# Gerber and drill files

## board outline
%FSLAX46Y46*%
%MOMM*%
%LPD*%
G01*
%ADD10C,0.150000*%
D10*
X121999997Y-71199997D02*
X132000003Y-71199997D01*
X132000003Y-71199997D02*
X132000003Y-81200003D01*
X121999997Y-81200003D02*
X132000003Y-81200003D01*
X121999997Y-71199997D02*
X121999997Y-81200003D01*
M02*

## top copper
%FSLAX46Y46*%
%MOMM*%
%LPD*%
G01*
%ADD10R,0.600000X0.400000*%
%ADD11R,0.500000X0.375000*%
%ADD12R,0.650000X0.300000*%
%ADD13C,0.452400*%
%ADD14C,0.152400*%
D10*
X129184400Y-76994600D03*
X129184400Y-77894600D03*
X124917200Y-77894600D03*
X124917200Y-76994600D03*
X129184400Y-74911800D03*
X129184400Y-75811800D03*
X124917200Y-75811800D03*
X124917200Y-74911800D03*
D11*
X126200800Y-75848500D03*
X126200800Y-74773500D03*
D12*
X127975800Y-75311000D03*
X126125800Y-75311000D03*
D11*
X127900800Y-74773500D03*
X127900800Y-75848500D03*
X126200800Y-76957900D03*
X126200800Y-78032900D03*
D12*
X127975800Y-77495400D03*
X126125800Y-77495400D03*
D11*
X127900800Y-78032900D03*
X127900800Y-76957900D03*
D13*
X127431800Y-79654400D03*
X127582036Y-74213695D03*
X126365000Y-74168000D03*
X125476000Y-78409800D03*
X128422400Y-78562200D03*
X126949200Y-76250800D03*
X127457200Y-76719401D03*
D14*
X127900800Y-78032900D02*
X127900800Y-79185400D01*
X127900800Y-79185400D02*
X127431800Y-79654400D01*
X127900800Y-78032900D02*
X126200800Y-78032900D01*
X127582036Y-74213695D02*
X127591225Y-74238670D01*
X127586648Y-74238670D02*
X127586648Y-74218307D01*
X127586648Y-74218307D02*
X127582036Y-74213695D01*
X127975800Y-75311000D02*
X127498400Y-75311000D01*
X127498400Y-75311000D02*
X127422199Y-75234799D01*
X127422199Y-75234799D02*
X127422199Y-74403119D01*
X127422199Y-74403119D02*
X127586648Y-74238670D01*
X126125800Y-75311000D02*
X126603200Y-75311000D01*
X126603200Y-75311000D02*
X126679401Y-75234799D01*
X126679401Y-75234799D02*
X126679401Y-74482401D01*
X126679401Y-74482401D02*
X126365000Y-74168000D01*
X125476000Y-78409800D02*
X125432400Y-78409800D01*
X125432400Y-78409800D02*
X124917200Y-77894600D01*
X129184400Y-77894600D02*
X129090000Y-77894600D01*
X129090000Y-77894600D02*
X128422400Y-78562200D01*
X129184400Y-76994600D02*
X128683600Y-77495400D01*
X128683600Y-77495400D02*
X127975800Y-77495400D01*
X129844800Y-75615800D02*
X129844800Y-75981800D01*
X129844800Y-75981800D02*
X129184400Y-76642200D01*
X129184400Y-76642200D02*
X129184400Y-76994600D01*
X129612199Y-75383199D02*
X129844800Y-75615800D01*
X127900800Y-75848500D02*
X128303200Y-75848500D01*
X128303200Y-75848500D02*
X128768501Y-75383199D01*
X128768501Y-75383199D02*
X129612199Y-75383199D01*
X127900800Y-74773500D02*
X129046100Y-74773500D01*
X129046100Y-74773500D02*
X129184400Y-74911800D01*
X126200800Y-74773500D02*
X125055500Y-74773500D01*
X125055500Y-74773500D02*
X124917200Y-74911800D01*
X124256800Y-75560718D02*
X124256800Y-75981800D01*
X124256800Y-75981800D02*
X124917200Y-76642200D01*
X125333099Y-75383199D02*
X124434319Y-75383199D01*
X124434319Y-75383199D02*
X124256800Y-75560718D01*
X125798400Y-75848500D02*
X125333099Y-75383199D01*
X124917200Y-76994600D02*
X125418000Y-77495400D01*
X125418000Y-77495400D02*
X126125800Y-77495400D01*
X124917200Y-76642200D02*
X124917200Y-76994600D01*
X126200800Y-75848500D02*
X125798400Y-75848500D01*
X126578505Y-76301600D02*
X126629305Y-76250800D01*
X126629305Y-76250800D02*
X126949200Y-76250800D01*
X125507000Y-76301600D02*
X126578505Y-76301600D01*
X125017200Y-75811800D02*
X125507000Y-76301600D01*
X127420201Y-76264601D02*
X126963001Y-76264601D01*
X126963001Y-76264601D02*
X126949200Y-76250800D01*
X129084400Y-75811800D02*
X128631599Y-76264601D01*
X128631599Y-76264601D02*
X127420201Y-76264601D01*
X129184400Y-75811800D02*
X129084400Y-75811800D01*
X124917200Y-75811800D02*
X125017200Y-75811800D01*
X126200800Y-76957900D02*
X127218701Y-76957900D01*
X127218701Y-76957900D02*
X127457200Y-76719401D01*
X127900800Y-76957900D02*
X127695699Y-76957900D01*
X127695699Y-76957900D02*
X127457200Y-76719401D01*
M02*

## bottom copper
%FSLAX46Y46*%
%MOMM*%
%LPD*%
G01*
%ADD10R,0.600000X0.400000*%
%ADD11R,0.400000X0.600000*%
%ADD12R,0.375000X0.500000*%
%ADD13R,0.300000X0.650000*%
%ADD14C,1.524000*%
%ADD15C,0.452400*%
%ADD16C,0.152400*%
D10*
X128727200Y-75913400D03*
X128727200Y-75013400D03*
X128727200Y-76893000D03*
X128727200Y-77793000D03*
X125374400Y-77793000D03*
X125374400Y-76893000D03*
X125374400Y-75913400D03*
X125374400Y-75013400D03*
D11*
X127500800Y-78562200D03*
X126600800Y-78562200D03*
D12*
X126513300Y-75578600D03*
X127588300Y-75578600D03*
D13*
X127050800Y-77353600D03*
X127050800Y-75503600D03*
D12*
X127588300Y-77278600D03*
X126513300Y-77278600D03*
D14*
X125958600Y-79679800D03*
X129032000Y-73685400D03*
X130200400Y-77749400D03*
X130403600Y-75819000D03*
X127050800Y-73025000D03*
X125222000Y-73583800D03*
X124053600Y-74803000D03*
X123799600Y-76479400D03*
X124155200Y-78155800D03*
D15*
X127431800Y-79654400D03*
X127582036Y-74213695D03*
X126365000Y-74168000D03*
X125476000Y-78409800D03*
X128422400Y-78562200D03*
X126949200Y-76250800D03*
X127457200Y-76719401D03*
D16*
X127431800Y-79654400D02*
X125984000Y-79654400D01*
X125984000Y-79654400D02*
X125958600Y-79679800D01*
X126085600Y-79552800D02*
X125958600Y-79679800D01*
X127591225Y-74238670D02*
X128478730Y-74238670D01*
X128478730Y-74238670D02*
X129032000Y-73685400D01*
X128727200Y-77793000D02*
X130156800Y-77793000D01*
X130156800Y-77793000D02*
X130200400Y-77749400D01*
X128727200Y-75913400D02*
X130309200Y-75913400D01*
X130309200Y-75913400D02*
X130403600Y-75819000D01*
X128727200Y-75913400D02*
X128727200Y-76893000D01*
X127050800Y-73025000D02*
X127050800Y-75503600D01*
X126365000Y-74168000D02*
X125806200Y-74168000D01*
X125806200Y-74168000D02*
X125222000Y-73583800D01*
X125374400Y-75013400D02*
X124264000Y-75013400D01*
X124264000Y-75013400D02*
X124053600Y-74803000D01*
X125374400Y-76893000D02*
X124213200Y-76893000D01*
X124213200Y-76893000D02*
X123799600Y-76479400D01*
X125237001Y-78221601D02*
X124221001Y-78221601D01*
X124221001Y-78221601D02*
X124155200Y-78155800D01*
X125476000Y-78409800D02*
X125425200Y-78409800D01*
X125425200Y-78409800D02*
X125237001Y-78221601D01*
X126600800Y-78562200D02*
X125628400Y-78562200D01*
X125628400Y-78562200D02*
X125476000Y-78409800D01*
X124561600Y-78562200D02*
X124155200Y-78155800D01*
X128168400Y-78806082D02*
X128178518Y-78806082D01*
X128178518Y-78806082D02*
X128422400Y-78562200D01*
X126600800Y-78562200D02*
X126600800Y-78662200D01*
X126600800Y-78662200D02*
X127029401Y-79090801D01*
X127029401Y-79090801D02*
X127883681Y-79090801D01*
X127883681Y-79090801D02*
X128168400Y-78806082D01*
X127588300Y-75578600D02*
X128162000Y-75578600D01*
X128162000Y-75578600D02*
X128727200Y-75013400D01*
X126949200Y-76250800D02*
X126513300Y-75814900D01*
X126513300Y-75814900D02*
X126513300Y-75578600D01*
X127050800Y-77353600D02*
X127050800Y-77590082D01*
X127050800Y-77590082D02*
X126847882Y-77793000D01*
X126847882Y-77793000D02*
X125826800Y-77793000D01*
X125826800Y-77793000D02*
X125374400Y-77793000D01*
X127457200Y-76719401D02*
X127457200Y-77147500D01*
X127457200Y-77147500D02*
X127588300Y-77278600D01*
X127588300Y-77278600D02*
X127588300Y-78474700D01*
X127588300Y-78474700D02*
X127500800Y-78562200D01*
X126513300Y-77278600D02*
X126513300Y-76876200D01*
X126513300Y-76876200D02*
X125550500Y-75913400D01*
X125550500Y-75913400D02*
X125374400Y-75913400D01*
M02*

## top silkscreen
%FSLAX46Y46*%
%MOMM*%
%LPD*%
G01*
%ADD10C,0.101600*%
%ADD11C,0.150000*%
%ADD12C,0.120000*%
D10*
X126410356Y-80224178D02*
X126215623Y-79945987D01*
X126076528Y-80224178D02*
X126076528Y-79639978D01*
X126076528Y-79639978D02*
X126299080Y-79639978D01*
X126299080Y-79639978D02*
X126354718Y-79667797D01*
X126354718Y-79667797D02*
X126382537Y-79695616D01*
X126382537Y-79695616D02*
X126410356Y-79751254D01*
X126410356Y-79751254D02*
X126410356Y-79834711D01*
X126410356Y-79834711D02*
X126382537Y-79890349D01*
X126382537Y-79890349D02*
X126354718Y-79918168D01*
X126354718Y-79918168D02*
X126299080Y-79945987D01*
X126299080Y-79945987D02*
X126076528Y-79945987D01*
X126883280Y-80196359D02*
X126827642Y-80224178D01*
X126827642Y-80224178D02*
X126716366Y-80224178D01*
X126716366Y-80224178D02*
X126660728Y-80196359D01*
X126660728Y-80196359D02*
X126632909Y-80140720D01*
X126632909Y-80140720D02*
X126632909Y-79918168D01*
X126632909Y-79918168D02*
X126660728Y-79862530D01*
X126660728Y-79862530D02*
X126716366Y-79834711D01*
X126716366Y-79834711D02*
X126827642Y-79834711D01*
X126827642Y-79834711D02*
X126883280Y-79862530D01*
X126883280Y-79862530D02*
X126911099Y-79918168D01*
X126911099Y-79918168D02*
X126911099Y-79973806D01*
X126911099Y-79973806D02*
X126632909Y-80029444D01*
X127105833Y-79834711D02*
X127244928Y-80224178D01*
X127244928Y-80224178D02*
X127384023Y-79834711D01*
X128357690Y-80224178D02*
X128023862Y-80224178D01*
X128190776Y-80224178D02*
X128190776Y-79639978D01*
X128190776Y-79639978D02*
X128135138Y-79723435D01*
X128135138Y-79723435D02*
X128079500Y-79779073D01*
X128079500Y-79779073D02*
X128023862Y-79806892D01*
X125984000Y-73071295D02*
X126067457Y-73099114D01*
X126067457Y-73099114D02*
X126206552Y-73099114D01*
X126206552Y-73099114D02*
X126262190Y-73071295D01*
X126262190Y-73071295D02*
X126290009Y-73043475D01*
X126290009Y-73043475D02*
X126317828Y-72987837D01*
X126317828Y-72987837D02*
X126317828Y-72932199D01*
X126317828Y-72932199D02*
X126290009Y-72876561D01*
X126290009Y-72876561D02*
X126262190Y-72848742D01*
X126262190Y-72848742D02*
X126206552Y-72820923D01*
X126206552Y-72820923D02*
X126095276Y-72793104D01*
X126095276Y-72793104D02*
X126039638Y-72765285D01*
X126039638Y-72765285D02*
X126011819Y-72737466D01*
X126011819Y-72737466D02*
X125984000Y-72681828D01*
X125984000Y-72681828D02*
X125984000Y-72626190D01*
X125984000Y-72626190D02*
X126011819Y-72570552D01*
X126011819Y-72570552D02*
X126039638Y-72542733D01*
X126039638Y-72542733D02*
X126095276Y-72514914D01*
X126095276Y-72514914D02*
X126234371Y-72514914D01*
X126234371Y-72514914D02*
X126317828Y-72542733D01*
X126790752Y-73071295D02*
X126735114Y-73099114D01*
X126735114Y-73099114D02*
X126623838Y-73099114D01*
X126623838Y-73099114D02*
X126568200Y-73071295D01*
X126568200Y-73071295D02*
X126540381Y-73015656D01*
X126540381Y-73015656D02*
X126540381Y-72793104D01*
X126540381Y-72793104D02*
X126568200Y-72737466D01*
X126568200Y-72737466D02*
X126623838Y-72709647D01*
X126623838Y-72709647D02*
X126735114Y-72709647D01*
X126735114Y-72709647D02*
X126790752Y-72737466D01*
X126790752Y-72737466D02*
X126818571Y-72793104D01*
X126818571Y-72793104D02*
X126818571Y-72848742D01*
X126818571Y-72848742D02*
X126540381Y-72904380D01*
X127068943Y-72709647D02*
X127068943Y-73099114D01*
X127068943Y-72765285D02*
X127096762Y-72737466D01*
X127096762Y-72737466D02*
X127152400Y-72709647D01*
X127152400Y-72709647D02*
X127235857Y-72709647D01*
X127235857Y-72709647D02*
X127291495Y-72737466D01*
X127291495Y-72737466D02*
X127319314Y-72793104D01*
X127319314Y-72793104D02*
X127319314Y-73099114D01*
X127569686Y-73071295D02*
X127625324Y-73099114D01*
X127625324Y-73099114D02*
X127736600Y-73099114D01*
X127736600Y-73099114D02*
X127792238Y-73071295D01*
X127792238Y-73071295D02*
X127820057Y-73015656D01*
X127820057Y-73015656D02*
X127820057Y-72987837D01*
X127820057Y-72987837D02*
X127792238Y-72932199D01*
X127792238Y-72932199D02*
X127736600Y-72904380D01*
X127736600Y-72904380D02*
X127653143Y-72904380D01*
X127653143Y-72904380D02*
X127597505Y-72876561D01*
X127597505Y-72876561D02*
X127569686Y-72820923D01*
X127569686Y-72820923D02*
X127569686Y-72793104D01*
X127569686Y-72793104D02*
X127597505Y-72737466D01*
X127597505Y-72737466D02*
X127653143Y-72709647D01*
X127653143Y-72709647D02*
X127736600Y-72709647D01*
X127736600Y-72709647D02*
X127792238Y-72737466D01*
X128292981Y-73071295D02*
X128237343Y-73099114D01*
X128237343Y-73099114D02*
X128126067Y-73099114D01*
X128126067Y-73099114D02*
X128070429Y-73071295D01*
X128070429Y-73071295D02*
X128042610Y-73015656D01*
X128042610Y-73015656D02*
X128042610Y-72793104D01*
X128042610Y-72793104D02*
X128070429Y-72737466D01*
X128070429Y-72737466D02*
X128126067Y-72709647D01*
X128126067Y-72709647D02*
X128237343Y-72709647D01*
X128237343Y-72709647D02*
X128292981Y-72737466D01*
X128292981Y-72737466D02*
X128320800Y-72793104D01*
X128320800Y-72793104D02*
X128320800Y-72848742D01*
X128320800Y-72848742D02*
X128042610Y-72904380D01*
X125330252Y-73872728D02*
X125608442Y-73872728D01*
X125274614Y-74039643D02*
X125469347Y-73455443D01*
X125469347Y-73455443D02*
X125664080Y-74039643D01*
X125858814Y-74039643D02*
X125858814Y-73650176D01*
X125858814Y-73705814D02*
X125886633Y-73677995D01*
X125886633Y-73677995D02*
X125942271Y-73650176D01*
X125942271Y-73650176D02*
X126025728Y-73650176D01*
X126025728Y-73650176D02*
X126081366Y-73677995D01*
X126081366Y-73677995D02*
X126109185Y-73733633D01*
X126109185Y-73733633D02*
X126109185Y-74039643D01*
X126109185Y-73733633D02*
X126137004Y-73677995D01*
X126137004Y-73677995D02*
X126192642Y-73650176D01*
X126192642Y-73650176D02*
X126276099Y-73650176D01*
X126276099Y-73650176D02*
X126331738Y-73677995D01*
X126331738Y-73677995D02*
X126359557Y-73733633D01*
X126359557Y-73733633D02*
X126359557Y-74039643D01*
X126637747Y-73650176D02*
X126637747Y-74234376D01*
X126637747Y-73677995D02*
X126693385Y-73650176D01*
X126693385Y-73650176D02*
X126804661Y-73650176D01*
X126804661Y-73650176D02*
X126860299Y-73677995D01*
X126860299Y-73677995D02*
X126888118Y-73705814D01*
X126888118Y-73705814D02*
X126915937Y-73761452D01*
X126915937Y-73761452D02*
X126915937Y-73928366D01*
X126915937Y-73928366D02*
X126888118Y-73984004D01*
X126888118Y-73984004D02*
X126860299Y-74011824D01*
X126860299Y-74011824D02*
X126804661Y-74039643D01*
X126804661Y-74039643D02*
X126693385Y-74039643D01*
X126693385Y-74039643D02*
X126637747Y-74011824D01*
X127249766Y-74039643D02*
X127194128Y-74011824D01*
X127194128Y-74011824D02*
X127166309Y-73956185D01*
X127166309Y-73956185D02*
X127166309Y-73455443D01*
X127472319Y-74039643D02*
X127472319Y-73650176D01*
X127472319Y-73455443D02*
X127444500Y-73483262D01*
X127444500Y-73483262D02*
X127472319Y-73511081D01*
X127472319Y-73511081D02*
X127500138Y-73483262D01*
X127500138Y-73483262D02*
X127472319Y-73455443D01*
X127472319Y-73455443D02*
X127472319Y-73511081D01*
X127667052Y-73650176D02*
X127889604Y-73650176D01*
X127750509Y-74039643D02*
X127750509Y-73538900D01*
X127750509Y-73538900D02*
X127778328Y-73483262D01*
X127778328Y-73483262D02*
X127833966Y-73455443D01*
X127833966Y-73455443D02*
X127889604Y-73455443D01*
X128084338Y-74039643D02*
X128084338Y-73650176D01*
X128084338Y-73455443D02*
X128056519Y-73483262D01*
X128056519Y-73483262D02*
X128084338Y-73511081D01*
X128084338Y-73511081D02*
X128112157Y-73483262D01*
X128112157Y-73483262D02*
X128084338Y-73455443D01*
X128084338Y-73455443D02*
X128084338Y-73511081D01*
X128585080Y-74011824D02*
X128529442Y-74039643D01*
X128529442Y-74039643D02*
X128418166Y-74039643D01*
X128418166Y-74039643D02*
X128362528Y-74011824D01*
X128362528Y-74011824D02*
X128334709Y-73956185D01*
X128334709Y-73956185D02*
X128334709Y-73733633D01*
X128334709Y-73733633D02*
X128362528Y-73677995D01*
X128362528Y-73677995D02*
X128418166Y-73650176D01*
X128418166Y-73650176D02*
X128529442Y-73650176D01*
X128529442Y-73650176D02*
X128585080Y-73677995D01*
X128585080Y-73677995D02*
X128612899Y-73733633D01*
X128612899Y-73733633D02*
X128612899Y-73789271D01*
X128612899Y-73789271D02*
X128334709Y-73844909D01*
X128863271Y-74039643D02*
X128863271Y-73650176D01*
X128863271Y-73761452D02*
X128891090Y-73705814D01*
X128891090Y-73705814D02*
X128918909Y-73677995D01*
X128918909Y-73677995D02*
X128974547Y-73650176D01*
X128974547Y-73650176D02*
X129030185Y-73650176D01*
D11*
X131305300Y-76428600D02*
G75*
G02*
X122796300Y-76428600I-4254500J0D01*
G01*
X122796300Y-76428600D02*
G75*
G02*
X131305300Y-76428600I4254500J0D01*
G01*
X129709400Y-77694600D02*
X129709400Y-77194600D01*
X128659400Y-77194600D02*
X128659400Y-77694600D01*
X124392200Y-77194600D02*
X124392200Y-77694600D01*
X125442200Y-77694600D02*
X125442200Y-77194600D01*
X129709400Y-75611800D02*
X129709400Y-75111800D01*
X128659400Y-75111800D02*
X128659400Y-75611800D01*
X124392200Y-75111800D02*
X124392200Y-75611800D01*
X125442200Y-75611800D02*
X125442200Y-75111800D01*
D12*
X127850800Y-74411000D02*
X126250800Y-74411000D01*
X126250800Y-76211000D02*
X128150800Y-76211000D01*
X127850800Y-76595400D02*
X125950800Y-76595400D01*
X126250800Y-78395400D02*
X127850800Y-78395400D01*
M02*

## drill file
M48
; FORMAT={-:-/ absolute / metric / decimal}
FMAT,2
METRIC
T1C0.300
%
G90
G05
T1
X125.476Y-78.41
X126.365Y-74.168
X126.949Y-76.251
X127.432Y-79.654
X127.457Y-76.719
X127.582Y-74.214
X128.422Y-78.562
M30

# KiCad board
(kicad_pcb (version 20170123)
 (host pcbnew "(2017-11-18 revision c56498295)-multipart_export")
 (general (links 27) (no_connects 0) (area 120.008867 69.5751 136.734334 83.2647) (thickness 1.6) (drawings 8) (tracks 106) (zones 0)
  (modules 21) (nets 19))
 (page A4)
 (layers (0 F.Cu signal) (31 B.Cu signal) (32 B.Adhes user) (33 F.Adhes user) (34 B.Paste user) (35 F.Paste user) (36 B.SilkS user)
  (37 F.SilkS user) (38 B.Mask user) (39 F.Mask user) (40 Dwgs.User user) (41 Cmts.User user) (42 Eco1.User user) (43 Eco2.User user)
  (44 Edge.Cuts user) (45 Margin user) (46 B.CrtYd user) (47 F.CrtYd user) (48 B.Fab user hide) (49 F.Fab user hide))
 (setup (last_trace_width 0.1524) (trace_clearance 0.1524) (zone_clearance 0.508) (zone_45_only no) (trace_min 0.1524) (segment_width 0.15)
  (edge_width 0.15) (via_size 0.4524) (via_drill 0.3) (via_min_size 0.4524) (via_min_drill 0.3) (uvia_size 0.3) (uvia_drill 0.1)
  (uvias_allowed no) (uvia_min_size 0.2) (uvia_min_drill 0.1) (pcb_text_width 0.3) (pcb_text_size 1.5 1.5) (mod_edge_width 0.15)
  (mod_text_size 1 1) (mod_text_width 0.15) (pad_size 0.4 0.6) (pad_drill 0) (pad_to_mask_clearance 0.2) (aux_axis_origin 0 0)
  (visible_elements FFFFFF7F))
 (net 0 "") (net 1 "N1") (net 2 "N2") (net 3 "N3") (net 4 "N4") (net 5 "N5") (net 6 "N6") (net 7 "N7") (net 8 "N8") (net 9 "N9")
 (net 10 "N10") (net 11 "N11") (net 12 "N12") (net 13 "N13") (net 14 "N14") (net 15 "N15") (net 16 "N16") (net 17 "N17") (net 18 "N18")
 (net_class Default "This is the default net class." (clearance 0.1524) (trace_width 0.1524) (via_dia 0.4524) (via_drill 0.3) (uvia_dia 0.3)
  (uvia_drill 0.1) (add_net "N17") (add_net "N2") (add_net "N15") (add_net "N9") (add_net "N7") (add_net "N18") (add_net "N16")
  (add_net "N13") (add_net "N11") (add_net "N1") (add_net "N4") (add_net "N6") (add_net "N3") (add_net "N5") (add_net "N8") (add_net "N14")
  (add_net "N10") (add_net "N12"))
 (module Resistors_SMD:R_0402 (layer F.Cu) (at 129.1844 77.4446 90)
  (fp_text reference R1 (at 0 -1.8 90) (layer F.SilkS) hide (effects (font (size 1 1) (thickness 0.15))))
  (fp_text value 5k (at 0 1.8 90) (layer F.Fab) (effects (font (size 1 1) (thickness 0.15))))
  (fp_line (start -0.25 0.525) (end 0.25 0.525) (layer F.SilkS) (width 0.15))
  (fp_line (start 0.25 -0.525) (end -0.25 -0.525) (layer F.SilkS) (width 0.15))
  (pad 2 smd rect (at 0.45 0 90) (size 0.4 0.6) (layers F.Cu F.Paste F.Mask) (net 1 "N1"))
  (pad 1 smd rect (at -0.45 0 90) (size 0.4 0.6) (layers F.Cu F.Paste F.Mask) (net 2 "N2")))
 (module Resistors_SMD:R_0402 (layer F.Cu) (at 124.9172 77.4446 90)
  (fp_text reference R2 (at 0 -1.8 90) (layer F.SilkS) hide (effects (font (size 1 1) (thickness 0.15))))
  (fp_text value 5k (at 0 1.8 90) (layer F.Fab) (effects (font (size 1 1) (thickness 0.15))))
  (fp_line (start 0.25 -0.525) (end -0.25 -0.525) (layer F.SilkS) (width 0.15))
  (fp_line (start -0.25 0.525) (end 0.25 0.525) (layer F.SilkS) (width 0.15))
  (pad 1 smd rect (at -0.45 0 90) (size 0.4 0.6) (layers F.Cu F.Paste F.Mask) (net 2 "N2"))
  (pad 2 smd rect (at 0.45 0 90) (size 0.4 0.6) (layers F.Cu F.Paste F.Mask) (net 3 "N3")))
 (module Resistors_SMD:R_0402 (layer F.Cu) (at 129.1844 75.3618 270)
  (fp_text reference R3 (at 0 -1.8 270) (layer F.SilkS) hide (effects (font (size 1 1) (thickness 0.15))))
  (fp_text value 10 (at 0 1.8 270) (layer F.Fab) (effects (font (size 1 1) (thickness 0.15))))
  (fp_line (start 0.25 -0.525) (end -0.25 -0.525) (layer F.SilkS) (width 0.15))
  (fp_line (start -0.25 0.525) (end 0.25 0.525) (layer F.SilkS) (width 0.15))
  (pad 1 smd rect (at -0.45 0 270) (size 0.4 0.6) (layers F.Cu F.Paste F.Mask) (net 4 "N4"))
  (pad 2 smd rect (at 0.45 0 270) (size 0.4 0.6) (layers F.Cu F.Paste F.Mask) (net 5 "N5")))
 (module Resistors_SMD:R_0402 (layer F.Cu) (at 124.9172 75.3618 270)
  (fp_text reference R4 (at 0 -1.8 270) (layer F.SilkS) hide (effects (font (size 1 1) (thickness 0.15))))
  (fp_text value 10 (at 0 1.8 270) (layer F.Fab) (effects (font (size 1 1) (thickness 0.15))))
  (fp_line (start -0.25 0.525) (end 0.25 0.525) (layer F.SilkS) (width 0.15))
  (fp_line (start 0.25 -0.525) (end -0.25 -0.525) (layer F.SilkS) (width 0.15))
  (pad 2 smd rect (at 0.45 0 270) (size 0.4 0.6) (layers F.Cu F.Paste F.Mask) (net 5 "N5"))
  (pad 1 smd rect (at -0.45 0 270) (size 0.4 0.6) (layers F.Cu F.Paste F.Mask) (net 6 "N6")))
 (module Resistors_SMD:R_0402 (layer B.Cu) (at 128.7272 75.4634 270)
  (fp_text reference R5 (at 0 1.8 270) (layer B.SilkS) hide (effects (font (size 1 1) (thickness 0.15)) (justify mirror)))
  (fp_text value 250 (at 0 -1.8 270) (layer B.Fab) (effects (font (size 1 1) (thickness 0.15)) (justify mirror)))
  (pad 2 smd rect (at 0.45 0 270) (size 0.4 0.6) (layers B.Cu B.Paste B.Mask) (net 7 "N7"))
  (pad 1 smd rect (at -0.45 0 270) (size 0.4 0.6) (layers B.Cu B.Paste B.Mask) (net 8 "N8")))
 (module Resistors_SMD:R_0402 (layer B.Cu) (at 128.7272 77.343 270)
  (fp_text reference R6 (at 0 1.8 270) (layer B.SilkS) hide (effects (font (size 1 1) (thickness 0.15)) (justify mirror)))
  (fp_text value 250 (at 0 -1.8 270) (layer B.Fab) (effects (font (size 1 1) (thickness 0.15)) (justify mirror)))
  (pad 1 smd rect (at -0.45 0 270) (size 0.4 0.6) (layers B.Cu B.Paste B.Mask) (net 7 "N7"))
  (pad 2 smd rect (at 0.45 0 270) (size 0.4 0.6) (layers B.Cu B.Paste B.Mask) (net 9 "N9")))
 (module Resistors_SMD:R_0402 (layer B.Cu) (at 125.3744 77.343 90)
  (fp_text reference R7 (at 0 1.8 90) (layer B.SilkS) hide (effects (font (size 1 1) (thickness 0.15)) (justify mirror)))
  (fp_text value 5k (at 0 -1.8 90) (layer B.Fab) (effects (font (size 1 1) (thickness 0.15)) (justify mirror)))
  (pad 1 smd rect (at -0.45 0 90) (size 0.4 0.6) (layers B.Cu B.Paste B.Mask) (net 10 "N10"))
  (pad 2 smd rect (at 0.45 0 90) (size 0.4 0.6) (layers B.Cu B.Paste B.Mask) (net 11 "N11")))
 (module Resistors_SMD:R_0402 (layer B.Cu) (at 125.3744 75.4634 90)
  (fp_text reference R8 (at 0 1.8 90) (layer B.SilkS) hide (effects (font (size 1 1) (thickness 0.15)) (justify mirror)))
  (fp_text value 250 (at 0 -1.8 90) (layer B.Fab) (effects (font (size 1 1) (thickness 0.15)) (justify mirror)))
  (pad 1 smd rect (at -0.45 0 90) (size 0.4 0.6) (layers B.Cu B.Paste B.Mask) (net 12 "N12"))
  (pad 2 smd rect (at 0.45 0 90) (size 0.4 0.6) (layers B.Cu B.Paste B.Mask) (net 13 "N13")))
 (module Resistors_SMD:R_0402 (layer B.Cu) (at 127.0508 78.5622)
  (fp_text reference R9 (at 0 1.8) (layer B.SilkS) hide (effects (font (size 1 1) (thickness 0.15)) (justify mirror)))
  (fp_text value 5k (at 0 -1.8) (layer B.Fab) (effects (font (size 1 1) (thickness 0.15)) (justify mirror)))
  (pad 2 smd rect (at 0.45 0) (size 0.4 0.6) (layers B.Cu B.Paste B.Mask) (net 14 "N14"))
  (pad 1 smd rect (at -0.45 0) (size 0.4 0.6) (layers B.Cu B.Paste B.Mask) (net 2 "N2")))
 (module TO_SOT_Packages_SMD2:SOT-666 (layer F.Cu) (at 127.0508 75.311 180)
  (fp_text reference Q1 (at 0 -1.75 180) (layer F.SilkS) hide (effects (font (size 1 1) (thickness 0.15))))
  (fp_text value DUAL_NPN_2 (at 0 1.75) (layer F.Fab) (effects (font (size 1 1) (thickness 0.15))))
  (fp_line (start -0.8 0.9) (end 0.8 0.9) (layer F.SilkS) (width 0.12))
  (fp_line (start 0.8 -0.9) (end -1.1 -0.9) (layer F.SilkS) (width 0.12))
  (pad 6 smd rect (at 0.85 -0.5375 180) (size 0.5 0.375) (layers F.Cu F.Paste F.Mask) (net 3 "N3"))
  (pad 4 smd rect (at 0.85 0.5375 180) (size 0.5 0.375) (layers F.Cu F.Paste F.Mask) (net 6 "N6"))
  (pad 2 smd rect (at -0.925 0 180) (size 0.65 0.3) (layers F.Cu F.Paste F.Mask) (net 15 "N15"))
  (pad 5 smd rect (at 0.925 0 180) (size 0.65 0.3) (layers F.Cu F.Paste F.Mask) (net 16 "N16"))
  (pad 3 smd rect (at -0.85 0.5375 180) (size 0.5 0.375) (layers F.Cu F.Paste F.Mask) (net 4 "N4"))
  (pad 1 smd rect (at -0.85 -0.5375 180) (size 0.5 0.375) (layers F.Cu F.Paste F.Mask) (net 1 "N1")))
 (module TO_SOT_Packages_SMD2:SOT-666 (layer F.Cu) (at 127.0508 77.4954)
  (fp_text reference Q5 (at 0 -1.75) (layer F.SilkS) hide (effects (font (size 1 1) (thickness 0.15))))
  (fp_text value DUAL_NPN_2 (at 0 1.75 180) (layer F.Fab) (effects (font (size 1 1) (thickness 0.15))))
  (fp_line (start 0.8 -0.9) (end -1.1 -0.9) (layer F.SilkS) (width 0.12))
  (fp_line (start -0.8 0.9) (end 0.8 0.9) (layer F.SilkS) (width 0.12))
  (pad 1 smd rect (at -0.85 -0.5375) (size 0.5 0.375) (layers F.Cu F.Paste F.Mask) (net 14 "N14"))
  (pad 3 smd rect (at -0.85 0.5375) (size 0.5 0.375) (layers F.Cu F.Paste F.Mask) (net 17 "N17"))
  (pad 5 smd rect (at 0.925 0) (size 0.65 0.3) (layers F.Cu F.Paste F.Mask) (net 1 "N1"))
  (pad 2 smd rect (at -0.925 0) (size 0.65 0.3) (layers F.Cu F.Paste F.Mask) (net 3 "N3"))
  (pad 4 smd rect (at 0.85 0.5375) (size 0.5 0.375) (layers F.Cu F.Paste F.Mask) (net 17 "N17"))
  (pad 6 smd rect (at 0.85 -0.5375) (size 0.5 0.375) (layers F.Cu F.Paste F.Mask) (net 14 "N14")))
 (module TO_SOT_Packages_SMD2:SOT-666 (layer B.Cu) (at 127.0508 76.4286 270)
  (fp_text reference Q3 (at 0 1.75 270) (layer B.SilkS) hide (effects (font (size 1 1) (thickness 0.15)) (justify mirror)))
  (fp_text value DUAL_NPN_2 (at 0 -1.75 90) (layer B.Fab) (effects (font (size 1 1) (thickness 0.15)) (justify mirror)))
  (pad 1 smd rect (at -0.85 0.5375 270) (size 0.5 0.375) (layers B.Cu B.Paste B.Mask) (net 5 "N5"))
  (pad 3 smd rect (at -0.85 -0.5375 270) (size 0.5 0.375) (layers B.Cu B.Paste B.Mask) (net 8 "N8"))
  (pad 5 smd rect (at 0.925 0 270) (size 0.65 0.3) (layers B.Cu B.Paste B.Mask) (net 10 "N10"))
  (pad 2 smd rect (at -0.925 0 270) (size 0.65 0.3) (layers B.Cu B.Paste B.Mask) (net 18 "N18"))
  (pad 4 smd rect (at 0.85 -0.5375 270) (size 0.5 0.375) (layers B.Cu B.Paste B.Mask) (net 14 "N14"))
  (pad 6 smd rect (at 0.85 0.5375 270) (size 0.5 0.375) (layers B.Cu B.Paste B.Mask) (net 12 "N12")))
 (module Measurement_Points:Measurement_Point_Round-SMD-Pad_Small (layer B.Cu) (at 125.9586 79.6798)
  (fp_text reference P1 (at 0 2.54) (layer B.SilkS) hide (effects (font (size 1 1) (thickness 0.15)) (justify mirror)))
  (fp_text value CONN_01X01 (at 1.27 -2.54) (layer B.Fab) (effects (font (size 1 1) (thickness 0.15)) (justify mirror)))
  (pad 1 smd circle (at 0 0) (size 1.524 1.524) (layers B.Cu B.Paste B.Mask) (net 17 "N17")))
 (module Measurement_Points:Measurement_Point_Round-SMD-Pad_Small (layer B.Cu) (at 129.032 73.6854)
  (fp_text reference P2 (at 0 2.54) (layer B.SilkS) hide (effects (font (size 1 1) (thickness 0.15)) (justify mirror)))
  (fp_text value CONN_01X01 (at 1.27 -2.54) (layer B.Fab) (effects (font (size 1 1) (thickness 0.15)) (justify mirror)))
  (pad 1 smd circle (at 0 0) (size 1.524 1.524) (layers B.Cu B.Paste B.Mask) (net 15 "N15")))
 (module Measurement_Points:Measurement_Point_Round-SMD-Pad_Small (layer B.Cu) (at 130.2004 77.7494)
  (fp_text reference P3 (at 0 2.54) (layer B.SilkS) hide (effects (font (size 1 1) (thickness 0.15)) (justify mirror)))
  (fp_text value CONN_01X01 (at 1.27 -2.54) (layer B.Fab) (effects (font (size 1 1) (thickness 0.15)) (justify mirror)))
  (pad 1 smd circle (at 0 0) (size 1.524 1.524) (layers B.Cu B.Paste B.Mask) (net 9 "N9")))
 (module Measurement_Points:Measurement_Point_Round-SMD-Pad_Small (layer B.Cu) (at 130.4036 75.819)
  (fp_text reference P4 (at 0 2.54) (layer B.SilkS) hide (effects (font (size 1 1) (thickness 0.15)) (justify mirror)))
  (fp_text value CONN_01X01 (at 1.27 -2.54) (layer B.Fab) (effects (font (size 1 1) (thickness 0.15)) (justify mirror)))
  (pad 1 smd circle (at 0 0) (size 1.524 1.524) (layers B.Cu B.Paste B.Mask) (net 7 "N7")))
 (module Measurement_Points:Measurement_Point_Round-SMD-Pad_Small (layer B.Cu) (at 127.0508 73.025)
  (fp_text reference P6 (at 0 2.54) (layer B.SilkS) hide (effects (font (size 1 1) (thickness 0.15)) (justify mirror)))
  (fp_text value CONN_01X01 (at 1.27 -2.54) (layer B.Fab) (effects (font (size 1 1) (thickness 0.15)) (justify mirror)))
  (pad 1 smd circle (at 0 0) (size 1.524 1.524) (layers B.Cu B.Paste B.Mask) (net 18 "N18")))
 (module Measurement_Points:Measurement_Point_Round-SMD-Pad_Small (layer B.Cu) (at 125.222 73.5838)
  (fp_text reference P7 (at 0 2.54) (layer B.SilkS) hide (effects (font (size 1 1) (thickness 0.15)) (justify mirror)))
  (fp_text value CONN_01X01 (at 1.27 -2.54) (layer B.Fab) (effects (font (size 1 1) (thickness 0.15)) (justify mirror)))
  (pad 1 smd circle (at 0 0) (size 1.524 1.524) (layers B.Cu B.Paste B.Mask) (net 16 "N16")))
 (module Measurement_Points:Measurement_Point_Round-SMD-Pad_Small (layer B.Cu) (at 124.0536 74.803)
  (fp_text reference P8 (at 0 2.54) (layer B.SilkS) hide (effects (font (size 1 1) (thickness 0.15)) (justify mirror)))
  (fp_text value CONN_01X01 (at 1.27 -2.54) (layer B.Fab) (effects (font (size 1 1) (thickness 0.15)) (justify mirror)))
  (pad 1 smd circle (at 0 0) (size 1.524 1.524) (layers B.Cu B.Paste B.Mask) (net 13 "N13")))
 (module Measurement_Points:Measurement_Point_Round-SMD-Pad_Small (layer B.Cu) (at 123.7996 76.4794)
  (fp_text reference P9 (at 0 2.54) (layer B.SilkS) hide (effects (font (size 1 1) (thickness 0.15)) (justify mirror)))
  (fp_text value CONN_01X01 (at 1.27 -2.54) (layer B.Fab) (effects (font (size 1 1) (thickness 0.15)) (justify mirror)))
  (pad 1 smd circle (at 0 0) (size 1.524 1.524) (layers B.Cu B.Paste B.Mask) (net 11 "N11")))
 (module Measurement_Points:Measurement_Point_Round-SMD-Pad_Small (layer B.Cu) (at 124.1552 78.1558)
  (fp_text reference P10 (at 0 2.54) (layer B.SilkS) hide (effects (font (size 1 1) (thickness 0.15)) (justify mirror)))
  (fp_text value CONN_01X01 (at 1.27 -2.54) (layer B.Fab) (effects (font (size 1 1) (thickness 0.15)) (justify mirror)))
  (pad 1 smd circle (at 0 0) (size 1.524 1.524) (layers B.Cu B.Paste B.Mask) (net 2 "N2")))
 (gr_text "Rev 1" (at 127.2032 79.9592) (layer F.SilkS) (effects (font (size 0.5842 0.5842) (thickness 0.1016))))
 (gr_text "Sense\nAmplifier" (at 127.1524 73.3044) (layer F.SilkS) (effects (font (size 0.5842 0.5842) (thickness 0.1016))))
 (gr_line (start 121.999997 71.199997) (end 132.000003 71.199997) (layer Edge.Cuts) (width 0.15))
 (gr_line (start 132.000003 71.199997) (end 132.000003 81.200003) (layer Edge.Cuts) (width 0.15))
 (gr_line (start 121.999997 81.200003) (end 132.000003 81.200003) (layer Edge.Cuts) (width 0.15))
 (gr_line (start 121.999997 71.199997) (end 121.999997 81.200003) (layer Edge.Cuts) (width 0.15))
 (gr_circle (center 127.0508 76.4286) (end 131.3053 76.4286) (layer F.SilkS) (width 0.15))
 (segment (start 127.4318 79.6544) (end 125.984 79.6544) (width 0.1524) (layer B.Cu) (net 17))
 (segment (start 125.984 79.6544) (end 125.9586 79.6798) (width 0.1524) (layer B.Cu) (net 17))
 (segment (start 127.9008 78.0329) (end 127.9008 79.1854) (width 0.1524) (layer F.Cu) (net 17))
 (segment (start 127.9008 79.1854) (end 127.4318 79.6544) (width 0.1524) (layer F.Cu) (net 17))
 (via (at 127.4318 79.6544) (size 0.4524) (drill 0.3) (layers F.Cu B.Cu) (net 17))
 (segment (start 126.0856 79.5528) (end 125.9586 79.6798) (width 0.1524) (layer B.Cu) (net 17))
 (segment (start 127.9008 78.0329) (end 126.2008 78.0329) (width 0.1524) (layer F.Cu) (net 17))
 (segment (start 127.582036 74.213695) (end 127.591225 74.23867) (width 0.1524) (layer F.Cu) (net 15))
 (segment (start 127.586648 74.23867) (end 127.586648 74.218307) (width 0.1524) (layer F.Cu) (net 15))
 (segment (start 127.586648 74.218307) (end 127.582036 74.213695) (width 0.1524) (layer F.Cu) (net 15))
 (via (at 127.582036 74.213695) (size 0.4524) (drill 0.3) (layers F.Cu B.Cu) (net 15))
 (segment (start 127.591225 74.23867) (end 128.47873 74.23867) (width 0.1524) (layer B.Cu) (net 15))
 (segment (start 128.47873 74.23867) (end 129.032 73.6854) (width 0.1524) (layer B.Cu) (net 15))
 (segment (start 127.9758 75.311) (end 127.4984 75.311) (width 0.1524) (layer F.Cu) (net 15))
 (segment (start 127.4984 75.311) (end 127.422199 75.234799) (width 0.1524) (layer F.Cu) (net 15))
 (segment (start 127.422199 75.234799) (end 127.422199 74.403119) (width 0.1524) (layer F.Cu) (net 15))
 (segment (start 127.422199 74.403119) (end 127.586648 74.23867) (width 0.1524) (layer F.Cu) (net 15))
 (segment (start 128.7272 77.793) (end 130.1568 77.793) (width 0.1524) (layer B.Cu) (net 9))
 (segment (start 130.1568 77.793) (end 130.2004 77.7494) (width 0.1524) (layer B.Cu) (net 9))
 (segment (start 128.7272 75.9134) (end 130.3092 75.9134) (width 0.1524) (layer B.Cu) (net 7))
 (segment (start 130.3092 75.9134) (end 130.4036 75.819) (width 0.1524) (layer B.Cu) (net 7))
 (segment (start 128.7272 75.9134) (end 128.7272 76.893) (width 0.1524) (layer B.Cu) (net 7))
 (segment (start 127.0508 73.025) (end 127.0508 75.5036) (width 0.1524) (layer B.Cu) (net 18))
 (via (at 126.365 74.168) (size 0.4524) (drill 0.3) (layers F.Cu B.Cu) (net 16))
 (segment (start 126.365 74.168) (end 125.8062 74.168) (width 0.1524) (layer B.Cu) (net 16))
 (segment (start 125.8062 74.168) (end 125.222 73.5838) (width 0.1524) (layer B.Cu) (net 16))
 (segment (start 126.1258 75.311) (end 126.6032 75.311) (width 0.1524) (layer F.Cu) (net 16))
 (segment (start 126.6032 75.311) (end 126.679401 75.234799) (width 0.1524) (layer F.Cu) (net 16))
 (segment (start 126.679401 75.234799) (end 126.679401 74.482401) (width 0.1524) (layer F.Cu) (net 16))
 (segment (start 126.679401 74.482401) (end 126.365 74.168) (width 0.1524) (layer F.Cu) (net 16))
 (segment (start 125.3744 75.0134) (end 124.264 75.0134) (width 0.1524) (layer B.Cu) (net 13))
 (segment (start 124.264 75.0134) (end 124.0536 74.803) (width 0.1524) (layer B.Cu) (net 13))
 (segment (start 125.3744 76.893) (end 124.2132 76.893) (width 0.1524) (layer B.Cu) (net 11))
 (segment (start 124.2132 76.893) (end 123.7996 76.4794) (width 0.1524) (layer B.Cu) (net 11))
 (segment (start 125.237001 78.221601) (end 124.221001 78.221601) (width 0.1524) (layer B.Cu) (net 2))
 (segment (start 124.221001 78.221601) (end 124.1552 78.1558) (width 0.1524) (layer B.Cu) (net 2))
 (segment (start 125.476 78.4098) (end 125.4252 78.4098) (width 0.1524) (layer B.Cu) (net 2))
 (segment (start 125.4252 78.4098) (end 125.237001 78.221601) (width 0.1524) (layer B.Cu) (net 2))
 (segment (start 125.476 78.4098) (end 125.4324 78.4098) (width 0.1524) (layer F.Cu) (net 2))
 (segment (start 125.4324 78.4098) (end 124.9172 77.8946) (width 0.1524) (layer F.Cu) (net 2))
 (segment (start 126.6008 78.5622) (end 125.6284 78.5622) (width 0.1524) (layer B.Cu) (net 2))
 (segment (start 125.6284 78.5622) (end 125.476 78.4098) (width 0.1524) (layer B.Cu) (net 2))
 (via (at 125.476 78.4098) (size 0.4524) (drill 0.3) (layers F.Cu B.Cu) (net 2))
 (via (at 128.4224 78.5622) (size 0.4524) (drill 0.3) (layers F.Cu B.Cu) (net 2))
 (segment (start 124.5616 78.5622) (end 124.1552 78.1558) (width 0.1524) (layer B.Cu) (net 2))
 (segment (start 129.1844 77.8946) (end 129.09 77.8946) (width 0.1524) (layer F.Cu) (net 2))
 (segment (start 129.09 77.8946) (end 128.4224 78.5622) (width 0.1524) (layer F.Cu) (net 2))
 (segment (start 128.1684 78.806082) (end 128.178518 78.806082) (width 0.1524) (layer B.Cu) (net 2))
 (segment (start 128.178518 78.806082) (end 128.4224 78.5622) (width 0.1524) (layer B.Cu) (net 2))
 (segment (start 126.6008 78.5622) (end 126.6008 78.6622) (width 0.1524) (layer B.Cu) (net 2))
 (segment (start 126.6008 78.6622) (end 127.029401 79.090801) (width 0.1524) (layer B.Cu) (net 2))
 (segment (start 127.029401 79.090801) (end 127.883681 79.090801) (width 0.1524) (layer B.Cu) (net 2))
 (segment (start 127.883681 79.090801) (end 128.1684 78.806082) (width 0.1524) (layer B.Cu) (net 2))
 (segment (start 129.1844 76.9946) (end 128.6836 77.4954) (width 0.1524) (layer F.Cu) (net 1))
 (segment (start 128.6836 77.4954) (end 127.9758 77.4954) (width 0.1524) (layer F.Cu) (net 1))
 (segment (start 129.8448 75.6158) (end 129.8448 75.9818) (width 0.1524) (layer F.Cu) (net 1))
 (segment (start 129.8448 75.9818) (end 129.1844 76.6422) (width 0.1524) (layer F.Cu) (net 1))
 (segment (start 129.1844 76.6422) (end 129.1844 76.9946) (width 0.1524) (layer F.Cu) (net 1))
 (segment (start 129.612199 75.383199) (end 129.8448 75.6158) (width 0.1524) (layer F.Cu) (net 1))
 (segment (start 127.9008 75.8485) (end 128.3032 75.8485) (width 0.1524) (layer F.Cu) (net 1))
 (segment (start 128.3032 75.8485) (end 128.768501 75.383199) (width 0.1524) (layer F.Cu) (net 1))
 (segment (start 128.768501 75.383199) (end 129.612199 75.383199) (width 0.1524) (layer F.Cu) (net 1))
 (segment (start 127.9008 74.7735) (end 129.0461 74.7735) (width 0.1524) (layer F.Cu) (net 4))
 (segment (start 129.0461 74.7735) (end 129.1844 74.9118) (width 0.1524) (layer F.Cu) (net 4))
 (segment (start 126.2008 74.7735) (end 125.0555 74.7735) (width 0.1524) (layer F.Cu) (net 6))
 (segment (start 125.0555 74.7735) (end 124.9172 74.9118) (width 0.1524) (layer F.Cu) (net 6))
 (segment (start 124.2568 75.560718) (end 124.2568 75.9818) (width 0.1524) (layer F.Cu) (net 3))
 (segment (start 124.2568 75.9818) (end 124.9172 76.6422) (width 0.1524) (layer F.Cu) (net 3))
 (segment (start 125.333099 75.383199) (end 124.434319 75.383199) (width 0.1524) (layer F.Cu) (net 3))
 (segment (start 124.434319 75.383199) (end 124.2568 75.560718) (width 0.1524) (layer F.Cu) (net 3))
 (segment (start 125.7984 75.8485) (end 125.333099 75.383199) (width 0.1524) (layer F.Cu) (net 3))
 (segment (start 124.9172 76.9946) (end 125.418 77.4954) (width 0.1524) (layer F.Cu) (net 3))
 (segment (start 125.418 77.4954) (end 126.1258 77.4954) (width 0.1524) (layer F.Cu) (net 3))
 (segment (start 124.9172 76.6422) (end 124.9172 76.9946) (width 0.1524) (layer F.Cu) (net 3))
 (segment (start 126.2008 75.8485) (end 125.7984 75.8485) (width 0.1524) (layer F.Cu) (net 3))
 (segment (start 127.5883 75.5786) (end 128.162 75.5786) (width 0.1524) (layer B.Cu) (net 8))
 (segment (start 128.162 75.5786) (end 128.7272 75.0134) (width 0.1524) (layer B.Cu) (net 8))
 (segment (start 126.578505 76.3016) (end 126.629305 76.2508) (width 0.1524) (layer F.Cu) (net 5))
 (segment (start 126.629305 76.2508) (end 126.9492 76.2508) (width 0.1524) (layer F.Cu) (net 5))
 (segment (start 125.507 76.3016) (end 126.578505 76.3016) (width 0.1524) (layer F.Cu) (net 5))
 (segment (start 125.0172 75.8118) (end 125.507 76.3016) (width 0.1524) (layer F.Cu) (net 5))
 (segment (start 126.9492 76.2508) (end 126.5133 75.8149) (width 0.1524) (layer B.Cu) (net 5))
 (segment (start 126.5133 75.8149) (end 126.5133 75.5786) (width 0.1524) (layer B.Cu) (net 5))
 (segment (start 127.420201 76.264601) (end 126.963001 76.264601) (width 0.1524) (layer F.Cu) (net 5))
 (segment (start 126.963001 76.264601) (end 126.9492 76.2508) (width 0.1524) (layer F.Cu) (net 5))
 (via (at 126.9492 76.2508) (size 0.4524) (drill 0.3) (layers F.Cu B.Cu) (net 5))
 (segment (start 129.0844 75.8118) (end 128.631599 76.264601) (width 0.1524) (layer F.Cu) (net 5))
 (segment (start 128.631599 76.264601) (end 127.420201 76.264601) (width 0.1524) (layer F.Cu) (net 5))
 (segment (start 129.1844 75.8118) (end 129.0844 75.8118) (width 0.1524) (layer F.Cu) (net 5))
 (segment (start 124.9172 75.8118) (end 125.0172 75.8118) (width 0.1524) (layer F.Cu) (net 5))
 (segment (start 127.0508 77.3536) (end 127.0508 77.590082) (width 0.1524) (layer B.Cu) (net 10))
 (segment (start 127.0508 77.590082) (end 126.847882 77.793) (width 0.1524) (layer B.Cu) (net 10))
 (segment (start 126.847882 77.793) (end 125.8268 77.793) (width 0.1524) (layer B.Cu) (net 10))
 (segment (start 125.8268 77.793) (end 125.3744 77.793) (width 0.1524) (layer B.Cu) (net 10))
 (segment (start 126.2008 76.9579) (end 127.218701 76.9579) (width 0.1524) (layer F.Cu) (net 14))
 (segment (start 127.218701 76.9579) (end 127.4572 76.719401) (width 0.1524) (layer F.Cu) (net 14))
 (segment (start 127.4572 76.719401) (end 127.4572 77.1475) (width 0.1524) (layer B.Cu) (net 14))
 (segment (start 127.4572 77.1475) (end 127.5883 77.2786) (width 0.1524) (layer B.Cu) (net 14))
 (segment (start 127.9008 76.9579) (end 127.695699 76.9579) (width 0.1524) (layer F.Cu) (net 14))
 (segment (start 127.695699 76.9579) (end 127.4572 76.719401) (width 0.1524) (layer F.Cu) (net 14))
 (via (at 127.4572 76.719401) (size 0.4524) (drill 0.3) (layers F.Cu B.Cu) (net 14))
 (segment (start 127.5883 77.2786) (end 127.5883 78.4747) (width 0.1524) (layer B.Cu) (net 14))
 (segment (start 127.5883 78.4747) (end 127.5008 78.5622) (width 0.1524) (layer B.Cu) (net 14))
 (segment (start 126.5133 77.2786) (end 126.5133 76.8762) (width 0.1524) (layer B.Cu) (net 12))
 (segment (start 126.5133 76.8762) (end 125.5505 75.9134) (width 0.1524) (layer B.Cu) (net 12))
 (segment (start 125.5505 75.9134) (end 125.3744 75.9134) (width 0.1524) (layer B.Cu) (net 12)))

